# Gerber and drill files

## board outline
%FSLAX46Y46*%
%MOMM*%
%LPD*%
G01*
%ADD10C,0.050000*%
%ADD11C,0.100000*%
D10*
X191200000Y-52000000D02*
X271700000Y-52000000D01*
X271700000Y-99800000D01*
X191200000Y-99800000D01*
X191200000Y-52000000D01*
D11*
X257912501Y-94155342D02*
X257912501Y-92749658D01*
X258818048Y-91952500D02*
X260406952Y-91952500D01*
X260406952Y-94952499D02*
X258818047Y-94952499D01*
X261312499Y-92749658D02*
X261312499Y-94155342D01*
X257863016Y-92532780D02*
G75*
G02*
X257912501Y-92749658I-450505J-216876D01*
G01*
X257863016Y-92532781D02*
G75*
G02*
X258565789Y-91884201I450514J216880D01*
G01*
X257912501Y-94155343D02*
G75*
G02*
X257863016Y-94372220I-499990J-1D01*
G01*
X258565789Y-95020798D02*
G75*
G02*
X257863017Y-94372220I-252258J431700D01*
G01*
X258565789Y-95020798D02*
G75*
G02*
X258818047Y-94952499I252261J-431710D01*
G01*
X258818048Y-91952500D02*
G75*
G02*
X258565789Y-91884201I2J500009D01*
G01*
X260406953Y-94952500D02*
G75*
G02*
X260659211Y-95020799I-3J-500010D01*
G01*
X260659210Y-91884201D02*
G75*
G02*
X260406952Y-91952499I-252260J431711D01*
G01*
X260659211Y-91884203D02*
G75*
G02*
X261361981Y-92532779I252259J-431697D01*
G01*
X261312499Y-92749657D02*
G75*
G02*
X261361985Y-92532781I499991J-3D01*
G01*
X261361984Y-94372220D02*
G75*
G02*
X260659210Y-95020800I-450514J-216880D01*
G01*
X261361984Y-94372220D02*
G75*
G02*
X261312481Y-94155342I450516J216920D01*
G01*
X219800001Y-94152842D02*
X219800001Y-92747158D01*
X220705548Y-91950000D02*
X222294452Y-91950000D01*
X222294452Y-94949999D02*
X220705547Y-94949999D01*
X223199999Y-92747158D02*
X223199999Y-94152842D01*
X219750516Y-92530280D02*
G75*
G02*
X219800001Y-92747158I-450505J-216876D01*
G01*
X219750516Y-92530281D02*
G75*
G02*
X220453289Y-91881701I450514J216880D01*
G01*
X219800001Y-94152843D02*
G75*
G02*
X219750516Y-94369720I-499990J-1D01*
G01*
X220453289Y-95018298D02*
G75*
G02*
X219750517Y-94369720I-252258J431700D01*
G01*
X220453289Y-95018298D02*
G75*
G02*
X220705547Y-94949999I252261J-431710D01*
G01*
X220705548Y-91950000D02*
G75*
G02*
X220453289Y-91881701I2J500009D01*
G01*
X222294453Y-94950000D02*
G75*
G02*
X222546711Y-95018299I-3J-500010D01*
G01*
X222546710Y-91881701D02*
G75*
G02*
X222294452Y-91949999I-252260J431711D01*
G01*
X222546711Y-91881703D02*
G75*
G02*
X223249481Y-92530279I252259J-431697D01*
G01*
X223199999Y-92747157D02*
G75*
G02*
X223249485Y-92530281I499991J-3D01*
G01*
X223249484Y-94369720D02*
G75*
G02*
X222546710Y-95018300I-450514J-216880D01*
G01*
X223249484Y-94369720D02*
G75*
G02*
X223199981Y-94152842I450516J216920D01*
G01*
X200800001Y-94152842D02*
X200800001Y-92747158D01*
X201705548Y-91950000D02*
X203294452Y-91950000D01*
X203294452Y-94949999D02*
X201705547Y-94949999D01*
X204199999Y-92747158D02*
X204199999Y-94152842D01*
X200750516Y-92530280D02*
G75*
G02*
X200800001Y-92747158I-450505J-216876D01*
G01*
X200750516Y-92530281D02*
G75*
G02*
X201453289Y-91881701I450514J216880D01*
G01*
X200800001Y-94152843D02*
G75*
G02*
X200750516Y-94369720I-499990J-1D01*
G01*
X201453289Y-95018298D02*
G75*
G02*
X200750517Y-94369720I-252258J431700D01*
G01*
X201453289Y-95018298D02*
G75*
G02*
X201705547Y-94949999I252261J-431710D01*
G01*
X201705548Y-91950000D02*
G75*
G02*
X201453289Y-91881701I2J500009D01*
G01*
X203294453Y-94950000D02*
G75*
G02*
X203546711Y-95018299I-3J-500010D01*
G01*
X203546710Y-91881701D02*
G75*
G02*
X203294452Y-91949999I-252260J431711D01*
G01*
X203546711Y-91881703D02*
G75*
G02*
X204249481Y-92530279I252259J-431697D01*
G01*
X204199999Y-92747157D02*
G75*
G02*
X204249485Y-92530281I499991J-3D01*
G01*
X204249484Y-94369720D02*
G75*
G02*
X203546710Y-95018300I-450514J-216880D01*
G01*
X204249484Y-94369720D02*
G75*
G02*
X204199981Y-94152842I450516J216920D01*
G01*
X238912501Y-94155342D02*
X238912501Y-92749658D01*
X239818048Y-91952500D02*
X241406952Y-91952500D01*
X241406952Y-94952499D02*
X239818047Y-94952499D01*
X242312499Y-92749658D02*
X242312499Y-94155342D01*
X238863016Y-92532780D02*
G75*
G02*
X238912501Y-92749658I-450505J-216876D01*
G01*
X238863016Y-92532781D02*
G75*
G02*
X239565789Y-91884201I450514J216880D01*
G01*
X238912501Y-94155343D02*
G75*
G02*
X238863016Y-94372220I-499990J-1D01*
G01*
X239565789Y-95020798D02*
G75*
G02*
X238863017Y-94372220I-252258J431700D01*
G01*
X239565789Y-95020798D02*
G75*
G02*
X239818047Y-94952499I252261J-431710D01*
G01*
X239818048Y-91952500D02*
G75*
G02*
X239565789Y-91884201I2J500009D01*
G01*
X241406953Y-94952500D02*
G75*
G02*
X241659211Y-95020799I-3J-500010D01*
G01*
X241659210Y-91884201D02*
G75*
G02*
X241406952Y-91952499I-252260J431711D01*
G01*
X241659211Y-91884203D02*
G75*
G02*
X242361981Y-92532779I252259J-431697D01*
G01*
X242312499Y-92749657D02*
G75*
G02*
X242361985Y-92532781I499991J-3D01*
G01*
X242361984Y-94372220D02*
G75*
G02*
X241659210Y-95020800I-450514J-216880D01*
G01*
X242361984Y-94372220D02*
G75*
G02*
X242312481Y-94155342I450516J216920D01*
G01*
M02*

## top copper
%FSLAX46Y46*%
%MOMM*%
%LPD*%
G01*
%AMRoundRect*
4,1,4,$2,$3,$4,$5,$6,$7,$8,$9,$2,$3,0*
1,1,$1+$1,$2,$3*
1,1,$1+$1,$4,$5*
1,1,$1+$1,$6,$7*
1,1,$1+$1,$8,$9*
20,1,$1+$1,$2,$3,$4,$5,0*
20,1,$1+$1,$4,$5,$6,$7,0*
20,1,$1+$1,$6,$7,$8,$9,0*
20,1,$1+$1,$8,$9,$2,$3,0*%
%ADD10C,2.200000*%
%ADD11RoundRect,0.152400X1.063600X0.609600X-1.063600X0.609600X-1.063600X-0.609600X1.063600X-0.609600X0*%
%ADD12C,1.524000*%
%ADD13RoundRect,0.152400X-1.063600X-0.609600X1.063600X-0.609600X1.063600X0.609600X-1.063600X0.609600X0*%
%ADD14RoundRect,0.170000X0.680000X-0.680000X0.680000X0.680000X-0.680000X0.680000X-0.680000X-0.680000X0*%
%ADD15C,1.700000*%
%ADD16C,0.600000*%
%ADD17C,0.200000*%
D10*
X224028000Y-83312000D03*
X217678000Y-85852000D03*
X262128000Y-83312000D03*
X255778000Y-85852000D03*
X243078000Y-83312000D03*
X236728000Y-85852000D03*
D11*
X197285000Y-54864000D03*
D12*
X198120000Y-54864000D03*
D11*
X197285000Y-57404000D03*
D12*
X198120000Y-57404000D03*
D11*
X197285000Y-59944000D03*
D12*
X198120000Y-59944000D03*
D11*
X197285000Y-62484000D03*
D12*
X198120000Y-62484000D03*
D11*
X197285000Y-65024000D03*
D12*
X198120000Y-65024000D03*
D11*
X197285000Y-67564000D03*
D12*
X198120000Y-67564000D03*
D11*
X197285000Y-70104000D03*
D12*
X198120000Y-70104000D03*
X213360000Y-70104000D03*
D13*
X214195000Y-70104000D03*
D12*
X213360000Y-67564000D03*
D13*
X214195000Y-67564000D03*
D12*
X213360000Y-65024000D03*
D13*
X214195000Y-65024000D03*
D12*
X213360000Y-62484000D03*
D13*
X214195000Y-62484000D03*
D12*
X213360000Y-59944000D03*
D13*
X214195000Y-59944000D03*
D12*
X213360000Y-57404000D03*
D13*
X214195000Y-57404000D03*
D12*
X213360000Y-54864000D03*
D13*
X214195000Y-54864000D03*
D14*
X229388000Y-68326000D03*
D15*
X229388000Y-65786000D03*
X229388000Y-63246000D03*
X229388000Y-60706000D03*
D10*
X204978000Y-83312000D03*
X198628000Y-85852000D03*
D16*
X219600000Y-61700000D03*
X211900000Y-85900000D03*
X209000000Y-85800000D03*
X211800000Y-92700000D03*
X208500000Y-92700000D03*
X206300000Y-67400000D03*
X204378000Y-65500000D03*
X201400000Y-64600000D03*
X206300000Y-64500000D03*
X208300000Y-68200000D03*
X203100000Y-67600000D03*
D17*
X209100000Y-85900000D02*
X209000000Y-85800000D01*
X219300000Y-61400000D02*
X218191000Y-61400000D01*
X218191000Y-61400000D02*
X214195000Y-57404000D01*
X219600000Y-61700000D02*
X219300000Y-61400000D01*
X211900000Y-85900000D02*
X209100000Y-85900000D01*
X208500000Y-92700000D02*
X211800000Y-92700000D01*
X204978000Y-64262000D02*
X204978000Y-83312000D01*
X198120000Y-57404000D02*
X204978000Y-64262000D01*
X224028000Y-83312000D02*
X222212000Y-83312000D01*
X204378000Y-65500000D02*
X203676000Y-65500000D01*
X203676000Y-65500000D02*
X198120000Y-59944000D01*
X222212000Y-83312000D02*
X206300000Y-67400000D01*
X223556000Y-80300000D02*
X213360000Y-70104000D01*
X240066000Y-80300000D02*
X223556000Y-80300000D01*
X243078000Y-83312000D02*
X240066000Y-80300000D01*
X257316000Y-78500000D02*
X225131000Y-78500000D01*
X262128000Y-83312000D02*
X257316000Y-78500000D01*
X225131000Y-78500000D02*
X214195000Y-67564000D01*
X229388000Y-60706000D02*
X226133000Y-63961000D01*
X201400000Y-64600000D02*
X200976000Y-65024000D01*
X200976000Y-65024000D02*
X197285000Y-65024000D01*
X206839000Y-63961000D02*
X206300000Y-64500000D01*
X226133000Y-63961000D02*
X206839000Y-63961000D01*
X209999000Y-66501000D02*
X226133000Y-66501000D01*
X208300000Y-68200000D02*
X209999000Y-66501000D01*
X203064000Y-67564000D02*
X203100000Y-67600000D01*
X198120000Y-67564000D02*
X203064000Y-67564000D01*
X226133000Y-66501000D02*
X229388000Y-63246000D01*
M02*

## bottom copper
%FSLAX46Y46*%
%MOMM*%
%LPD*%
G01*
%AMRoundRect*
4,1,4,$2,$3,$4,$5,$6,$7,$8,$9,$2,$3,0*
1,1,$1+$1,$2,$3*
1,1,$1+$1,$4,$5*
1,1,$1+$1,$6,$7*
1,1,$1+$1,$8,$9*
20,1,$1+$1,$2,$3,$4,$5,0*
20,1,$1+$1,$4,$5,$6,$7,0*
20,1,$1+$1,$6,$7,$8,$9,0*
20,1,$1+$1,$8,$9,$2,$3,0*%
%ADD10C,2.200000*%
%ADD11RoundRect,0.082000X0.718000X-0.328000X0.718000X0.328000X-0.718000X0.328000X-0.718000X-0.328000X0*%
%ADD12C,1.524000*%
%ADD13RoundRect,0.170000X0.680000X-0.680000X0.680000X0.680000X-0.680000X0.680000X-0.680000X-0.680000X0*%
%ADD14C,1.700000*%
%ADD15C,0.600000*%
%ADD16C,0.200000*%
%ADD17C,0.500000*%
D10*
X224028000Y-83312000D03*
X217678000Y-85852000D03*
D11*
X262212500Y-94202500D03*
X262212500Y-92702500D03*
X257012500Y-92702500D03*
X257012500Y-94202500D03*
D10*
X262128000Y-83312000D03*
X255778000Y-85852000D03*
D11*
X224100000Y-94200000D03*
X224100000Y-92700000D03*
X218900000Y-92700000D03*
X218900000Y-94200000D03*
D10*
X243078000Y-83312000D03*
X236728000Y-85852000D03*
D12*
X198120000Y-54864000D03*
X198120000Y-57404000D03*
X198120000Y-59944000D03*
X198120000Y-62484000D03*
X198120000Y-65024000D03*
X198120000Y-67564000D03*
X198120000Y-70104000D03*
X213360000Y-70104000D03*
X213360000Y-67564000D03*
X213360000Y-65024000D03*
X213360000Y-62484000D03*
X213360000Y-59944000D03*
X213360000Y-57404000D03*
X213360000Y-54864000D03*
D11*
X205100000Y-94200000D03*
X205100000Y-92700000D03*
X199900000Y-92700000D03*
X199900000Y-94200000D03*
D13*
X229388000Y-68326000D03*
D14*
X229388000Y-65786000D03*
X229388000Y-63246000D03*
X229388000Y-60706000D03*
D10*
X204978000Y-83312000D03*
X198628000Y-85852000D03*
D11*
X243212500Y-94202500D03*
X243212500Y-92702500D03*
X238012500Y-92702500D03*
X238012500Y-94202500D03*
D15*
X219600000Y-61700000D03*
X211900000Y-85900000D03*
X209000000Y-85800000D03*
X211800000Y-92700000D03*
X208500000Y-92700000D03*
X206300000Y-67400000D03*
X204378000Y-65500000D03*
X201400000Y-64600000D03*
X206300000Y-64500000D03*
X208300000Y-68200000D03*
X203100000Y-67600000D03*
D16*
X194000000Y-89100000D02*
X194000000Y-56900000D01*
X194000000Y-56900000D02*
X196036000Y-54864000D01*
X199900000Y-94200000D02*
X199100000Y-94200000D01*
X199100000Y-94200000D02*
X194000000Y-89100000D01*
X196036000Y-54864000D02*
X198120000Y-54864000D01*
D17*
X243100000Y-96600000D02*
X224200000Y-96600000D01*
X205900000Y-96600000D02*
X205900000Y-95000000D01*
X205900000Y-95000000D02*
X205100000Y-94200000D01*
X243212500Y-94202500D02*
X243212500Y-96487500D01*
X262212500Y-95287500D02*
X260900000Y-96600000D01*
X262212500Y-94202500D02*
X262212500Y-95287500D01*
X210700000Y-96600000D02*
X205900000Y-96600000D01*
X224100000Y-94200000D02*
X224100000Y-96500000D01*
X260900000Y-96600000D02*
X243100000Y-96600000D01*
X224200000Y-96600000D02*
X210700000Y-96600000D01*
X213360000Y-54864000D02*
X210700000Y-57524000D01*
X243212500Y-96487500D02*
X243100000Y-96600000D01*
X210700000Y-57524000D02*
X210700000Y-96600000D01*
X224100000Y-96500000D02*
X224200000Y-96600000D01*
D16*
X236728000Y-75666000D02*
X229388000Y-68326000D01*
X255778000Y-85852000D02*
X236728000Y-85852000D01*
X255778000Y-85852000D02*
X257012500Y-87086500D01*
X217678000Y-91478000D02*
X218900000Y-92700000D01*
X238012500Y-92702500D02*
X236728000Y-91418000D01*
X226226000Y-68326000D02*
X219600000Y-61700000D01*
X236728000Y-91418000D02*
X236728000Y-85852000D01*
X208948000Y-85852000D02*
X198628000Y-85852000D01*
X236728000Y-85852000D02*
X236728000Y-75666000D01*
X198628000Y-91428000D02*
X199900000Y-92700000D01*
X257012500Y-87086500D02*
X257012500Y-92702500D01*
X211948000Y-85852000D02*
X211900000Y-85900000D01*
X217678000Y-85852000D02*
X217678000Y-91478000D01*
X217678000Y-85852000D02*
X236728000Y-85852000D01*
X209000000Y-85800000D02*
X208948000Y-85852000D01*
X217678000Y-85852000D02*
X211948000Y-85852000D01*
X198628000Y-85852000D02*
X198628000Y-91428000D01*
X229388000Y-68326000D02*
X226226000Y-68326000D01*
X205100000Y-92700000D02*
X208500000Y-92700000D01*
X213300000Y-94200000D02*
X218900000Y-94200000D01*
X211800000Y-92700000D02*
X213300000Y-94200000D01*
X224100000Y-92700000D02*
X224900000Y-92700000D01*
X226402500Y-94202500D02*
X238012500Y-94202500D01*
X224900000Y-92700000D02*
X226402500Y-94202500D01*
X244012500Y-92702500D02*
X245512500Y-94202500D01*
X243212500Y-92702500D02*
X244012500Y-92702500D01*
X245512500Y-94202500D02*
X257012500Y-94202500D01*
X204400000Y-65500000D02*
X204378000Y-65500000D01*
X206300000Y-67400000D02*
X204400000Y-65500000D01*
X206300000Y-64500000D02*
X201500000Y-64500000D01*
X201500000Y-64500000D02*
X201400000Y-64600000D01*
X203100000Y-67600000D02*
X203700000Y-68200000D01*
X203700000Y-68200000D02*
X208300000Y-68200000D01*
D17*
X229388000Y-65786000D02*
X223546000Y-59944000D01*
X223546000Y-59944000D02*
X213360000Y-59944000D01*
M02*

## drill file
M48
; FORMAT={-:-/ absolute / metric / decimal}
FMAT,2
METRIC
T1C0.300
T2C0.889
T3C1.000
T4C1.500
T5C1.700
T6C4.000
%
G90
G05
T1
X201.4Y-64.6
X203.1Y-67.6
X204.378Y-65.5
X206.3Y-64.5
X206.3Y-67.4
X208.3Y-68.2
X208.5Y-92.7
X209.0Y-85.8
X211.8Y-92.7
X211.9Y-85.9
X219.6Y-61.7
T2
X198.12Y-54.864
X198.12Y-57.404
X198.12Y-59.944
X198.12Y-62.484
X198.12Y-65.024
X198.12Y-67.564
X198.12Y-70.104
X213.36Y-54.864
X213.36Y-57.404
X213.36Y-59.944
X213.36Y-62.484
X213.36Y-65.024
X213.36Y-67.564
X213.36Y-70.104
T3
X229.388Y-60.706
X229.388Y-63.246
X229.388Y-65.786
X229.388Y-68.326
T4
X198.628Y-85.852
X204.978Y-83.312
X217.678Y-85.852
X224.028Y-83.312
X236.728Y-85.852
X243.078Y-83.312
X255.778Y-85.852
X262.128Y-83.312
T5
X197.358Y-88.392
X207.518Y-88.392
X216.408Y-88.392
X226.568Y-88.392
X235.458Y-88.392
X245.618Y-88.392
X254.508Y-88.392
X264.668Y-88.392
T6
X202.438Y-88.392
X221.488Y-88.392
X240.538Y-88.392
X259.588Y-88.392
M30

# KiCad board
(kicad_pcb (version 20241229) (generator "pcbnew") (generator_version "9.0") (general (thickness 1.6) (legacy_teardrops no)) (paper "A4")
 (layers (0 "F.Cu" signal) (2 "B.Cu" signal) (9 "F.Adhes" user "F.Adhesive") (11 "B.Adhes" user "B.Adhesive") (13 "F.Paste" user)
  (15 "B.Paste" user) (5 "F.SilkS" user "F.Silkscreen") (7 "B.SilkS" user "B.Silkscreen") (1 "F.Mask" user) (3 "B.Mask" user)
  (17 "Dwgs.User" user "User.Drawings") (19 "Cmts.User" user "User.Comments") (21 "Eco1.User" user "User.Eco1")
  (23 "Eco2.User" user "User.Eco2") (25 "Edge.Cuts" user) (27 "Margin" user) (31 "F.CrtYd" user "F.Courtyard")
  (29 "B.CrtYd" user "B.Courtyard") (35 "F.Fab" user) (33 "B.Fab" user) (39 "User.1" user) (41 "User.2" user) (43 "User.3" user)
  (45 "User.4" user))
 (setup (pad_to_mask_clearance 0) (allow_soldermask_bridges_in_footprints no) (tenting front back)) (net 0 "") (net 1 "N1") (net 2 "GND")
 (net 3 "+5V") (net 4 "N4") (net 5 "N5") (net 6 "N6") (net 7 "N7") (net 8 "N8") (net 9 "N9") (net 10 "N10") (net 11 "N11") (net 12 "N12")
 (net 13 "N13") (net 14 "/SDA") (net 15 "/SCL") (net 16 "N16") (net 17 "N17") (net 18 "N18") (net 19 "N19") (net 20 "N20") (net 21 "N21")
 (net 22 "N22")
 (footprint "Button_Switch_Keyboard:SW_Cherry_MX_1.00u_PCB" (layer "F.Cu") (at 224.028 83.312)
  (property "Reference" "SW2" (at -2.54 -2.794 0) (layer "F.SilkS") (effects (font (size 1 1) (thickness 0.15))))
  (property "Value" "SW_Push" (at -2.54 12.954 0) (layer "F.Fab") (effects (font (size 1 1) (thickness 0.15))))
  (pad "" np_thru_hole circle (at -7.62 5.08) (size 1.7 1.7) (drill 1.7) (layers "*.Cu" "*.Mask"))
  (pad "" np_thru_hole circle (at -2.54 5.08) (size 4 4) (drill 4) (layers "*.Cu" "*.Mask"))
  (pad "" np_thru_hole circle (at 2.54 5.08) (size 1.7 1.7) (drill 1.7) (layers "*.Cu" "*.Mask"))
  (pad "1" thru_hole circle (at 0 0) (size 2.2 2.2) (drill 1.5) (layers "*.Cu" "*.Mask") (remove_unused_layers no) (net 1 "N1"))
  (pad "2" thru_hole circle (at -6.35 2.54) (size 2.2 2.2) (drill 1.5) (layers "*.Cu" "*.Mask") (remove_unused_layers no) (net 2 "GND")))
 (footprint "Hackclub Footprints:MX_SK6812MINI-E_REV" (layer "F.Cu") (at 259.6125 88.3725)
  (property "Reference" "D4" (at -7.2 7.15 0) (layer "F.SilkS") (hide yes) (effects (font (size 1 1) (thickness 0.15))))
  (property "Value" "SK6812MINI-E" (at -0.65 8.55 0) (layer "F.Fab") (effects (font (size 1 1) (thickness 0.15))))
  (fp_line (start -1.699999 5.782842) (end -1.699999 4.377158) (stroke (width 0.1) (type solid)) (layer "Edge.Cuts"))
  (fp_line (start -0.794452 3.58) (end 0.794452 3.58) (stroke (width 0.1) (type solid)) (layer "Edge.Cuts"))
  (fp_line (start 0.794452 6.579999) (end -0.794453 6.579999) (stroke (width 0.1) (type solid)) (layer "Edge.Cuts"))
  (fp_line (start 1.699999 4.377158) (end 1.699999 5.782842) (stroke (width 0.1) (type solid)) (layer "Edge.Cuts"))
  (fp_arc (start -1.749484 4.16028) (mid -1.712527 4.265932) (end -1.699999 4.377158) (stroke (width 0.1) (type solid)) (layer "Edge.Cuts"))
  (fp_arc (start -1.749484 4.160281) (mid -1.638072 3.575965) (end -1.046711 3.511701) (stroke (width 0.1) (type solid)) (layer "Edge.Cuts"))
  (fp_arc (start -1.699999 5.782843) (mid -1.712527 5.894068) (end -1.749484 5.99972) (stroke (width 0.1) (type solid)) (layer "Edge.Cuts"))
  (fp_arc (start -1.046711 6.648298) (mid -1.638071 6.584034) (end -1.749484 5.99972) (stroke (width 0.1) (type solid)) (layer "Edge.Cuts"))
  (fp_arc (start -1.046711 6.648298) (mid -0.925123 6.597376) (end -0.794453 6.579999) (stroke (width 0.1) (type solid)) (layer "Edge.Cuts"))
  (fp_arc (start -0.794452 3.58) (mid -0.925123 3.562623) (end -1.046711 3.511701) (stroke (width 0.1) (type solid)) (layer "Edge.Cuts"))
  (fp_arc (start 0.794453 6.58) (mid 0.925123 6.597377) (end 1.046711 6.648299) (stroke (width 0.1) (type solid)) (layer "Edge.Cuts"))
  (fp_arc (start 1.04671 3.511701) (mid 0.925122 3.562623) (end 0.794452 3.58) (stroke (width 0.1) (type solid)) (layer "Edge.Cuts"))
  (fp_arc (start 1.046711 3.511703) (mid 1.63807 3.575966) (end 1.749484 4.16028) (stroke (width 0.1) (type solid)) (layer "Edge.Cuts"))
  (fp_arc (start 1.699999 4.377157) (mid 1.712527 4.265932) (end 1.749484 4.16028) (stroke (width 0.1) (type solid)) (layer "Edge.Cuts"))
  (fp_arc (start 1.749484 5.99972) (mid 1.638071 6.584035) (end 1.046711 6.648299) (stroke (width 0.1) (type solid)) (layer "Edge.Cuts"))
  (fp_arc (start 1.749484 5.99972) (mid 1.712527 5.894068) (end 1.699999 5.782842) (stroke (width 0.1) (type solid)) (layer "Edge.Cuts"))
  (pad "1" smd roundrect (at 2.6 5.83 90) (size 0.82 1.6) (layers "B.Cu" "B.Mask" "B.Paste") (roundrect_rratio 0.1) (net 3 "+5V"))
  (pad "2" smd roundrect (at 2.6 4.33 90) (size 0.82 1.6) (layers "B.Cu" "B.Mask" "B.Paste") (roundrect_rratio 0.1) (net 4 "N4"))
  (pad "3" smd roundrect (at -2.6 4.33 90) (size 0.82 1.6) (layers "B.Cu" "B.Mask" "B.Paste") (roundrect_rratio 0.1) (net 2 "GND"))
  (pad "4" smd roundrect (at -2.6 5.83 90) (size 0.82 1.6) (layers "B.Cu" "B.Mask" "B.Paste") (roundrect_rratio 0.1) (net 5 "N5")))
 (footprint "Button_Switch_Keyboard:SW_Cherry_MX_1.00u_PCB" (layer "F.Cu") (at 262.128 83.312)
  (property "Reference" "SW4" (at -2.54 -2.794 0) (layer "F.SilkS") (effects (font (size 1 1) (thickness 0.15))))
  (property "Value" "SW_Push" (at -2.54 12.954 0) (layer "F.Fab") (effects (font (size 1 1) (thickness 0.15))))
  (pad "" np_thru_hole circle (at -7.62 5.08) (size 1.7 1.7) (drill 1.7) (layers "*.Cu" "*.Mask"))
  (pad "" np_thru_hole circle (at -2.54 5.08) (size 4 4) (drill 4) (layers "*.Cu" "*.Mask"))
  (pad "" np_thru_hole circle (at 2.54 5.08) (size 1.7 1.7) (drill 1.7) (layers "*.Cu" "*.Mask"))
  (pad "1" thru_hole circle (at 0 0) (size 2.2 2.2) (drill 1.5) (layers "*.Cu" "*.Mask") (remove_unused_layers no) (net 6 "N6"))
  (pad "2" thru_hole circle (at -6.35 2.54) (size 2.2 2.2) (drill 1.5) (layers "*.Cu" "*.Mask") (remove_unused_layers no) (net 2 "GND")))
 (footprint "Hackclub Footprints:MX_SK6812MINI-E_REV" (layer "F.Cu") (at 221.5 88.37)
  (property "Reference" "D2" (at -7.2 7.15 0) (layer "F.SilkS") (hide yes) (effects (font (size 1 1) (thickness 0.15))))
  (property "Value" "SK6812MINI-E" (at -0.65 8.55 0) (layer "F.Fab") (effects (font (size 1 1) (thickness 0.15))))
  (fp_line (start -1.699999 5.782842) (end -1.699999 4.377158) (stroke (width 0.1) (type solid)) (layer "Edge.Cuts"))
  (fp_line (start -0.794452 3.58) (end 0.794452 3.58) (stroke (width 0.1) (type solid)) (layer "Edge.Cuts"))
  (fp_line (start 0.794452 6.579999) (end -0.794453 6.579999) (stroke (width 0.1) (type solid)) (layer "Edge.Cuts"))
  (fp_line (start 1.699999 4.377158) (end 1.699999 5.782842) (stroke (width 0.1) (type solid)) (layer "Edge.Cuts"))
  (fp_arc (start -1.749484 4.16028) (mid -1.712527 4.265932) (end -1.699999 4.377158) (stroke (width 0.1) (type solid)) (layer "Edge.Cuts"))
  (fp_arc (start -1.749484 4.160281) (mid -1.638072 3.575965) (end -1.046711 3.511701) (stroke (width 0.1) (type solid)) (layer "Edge.Cuts"))
  (fp_arc (start -1.699999 5.782843) (mid -1.712527 5.894068) (end -1.749484 5.99972) (stroke (width 0.1) (type solid)) (layer "Edge.Cuts"))
  (fp_arc (start -1.046711 6.648298) (mid -1.638071 6.584034) (end -1.749484 5.99972) (stroke (width 0.1) (type solid)) (layer "Edge.Cuts"))
  (fp_arc (start -1.046711 6.648298) (mid -0.925123 6.597376) (end -0.794453 6.579999) (stroke (width 0.1) (type solid)) (layer "Edge.Cuts"))
  (fp_arc (start -0.794452 3.58) (mid -0.925123 3.562623) (end -1.046711 3.511701) (stroke (width 0.1) (type solid)) (layer "Edge.Cuts"))
  (fp_arc (start 0.794453 6.58) (mid 0.925123 6.597377) (end 1.046711 6.648299) (stroke (width 0.1) (type solid)) (layer "Edge.Cuts"))
  (fp_arc (start 1.04671 3.511701) (mid 0.925122 3.562623) (end 0.794452 3.58) (stroke (width 0.1) (type solid)) (layer "Edge.Cuts"))
  (fp_arc (start 1.046711 3.511703) (mid 1.63807 3.575966) (end 1.749484 4.16028) (stroke (width 0.1) (type solid)) (layer "Edge.Cuts"))
  (fp_arc (start 1.699999 4.377157) (mid 1.712527 4.265932) (end 1.749484 4.16028) (stroke (width 0.1) (type solid)) (layer "Edge.Cuts"))
  (fp_arc (start 1.749484 5.99972) (mid 1.638071 6.584035) (end 1.046711 6.648299) (stroke (width 0.1) (type solid)) (layer "Edge.Cuts"))
  (fp_arc (start 1.749484 5.99972) (mid 1.712527 5.894068) (end 1.699999 5.782842) (stroke (width 0.1) (type solid)) (layer "Edge.Cuts"))
  (pad "1" smd roundrect (at 2.6 5.83 90) (size 0.82 1.6) (layers "B.Cu" "B.Mask" "B.Paste") (roundrect_rratio 0.1) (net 3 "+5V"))
  (pad "2" smd roundrect (at 2.6 4.33 90) (size 0.82 1.6) (layers "B.Cu" "B.Mask" "B.Paste") (roundrect_rratio 0.1) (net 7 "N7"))
  (pad "3" smd roundrect (at -2.6 4.33 90) (size 0.82 1.6) (layers "B.Cu" "B.Mask" "B.Paste") (roundrect_rratio 0.1) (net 2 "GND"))
  (pad "4" smd roundrect (at -2.6 5.83 90) (size 0.82 1.6) (layers "B.Cu" "B.Mask" "B.Paste") (roundrect_rratio 0.1) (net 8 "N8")))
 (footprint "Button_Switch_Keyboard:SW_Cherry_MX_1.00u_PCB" (layer "F.Cu") (at 243.078 83.312)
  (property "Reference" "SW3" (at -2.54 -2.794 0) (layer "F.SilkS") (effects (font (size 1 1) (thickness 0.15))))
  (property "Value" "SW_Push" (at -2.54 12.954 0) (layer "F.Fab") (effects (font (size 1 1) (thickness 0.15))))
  (pad "" np_thru_hole circle (at -7.62 5.08) (size 1.7 1.7) (drill 1.7) (layers "*.Cu" "*.Mask"))
  (pad "" np_thru_hole circle (at -2.54 5.08) (size 4 4) (drill 4) (layers "*.Cu" "*.Mask"))
  (pad "" np_thru_hole circle (at 2.54 5.08) (size 1.7 1.7) (drill 1.7) (layers "*.Cu" "*.Mask"))
  (pad "1" thru_hole circle (at 0 0) (size 2.2 2.2) (drill 1.5) (layers "*.Cu" "*.Mask") (remove_unused_layers no) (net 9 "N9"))
  (pad "2" thru_hole circle (at -6.35 2.54) (size 2.2 2.2) (drill 1.5) (layers "*.Cu" "*.Mask") (remove_unused_layers no) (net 2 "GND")))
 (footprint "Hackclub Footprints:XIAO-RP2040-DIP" (layer "F.Cu") (at 205.74 62.484)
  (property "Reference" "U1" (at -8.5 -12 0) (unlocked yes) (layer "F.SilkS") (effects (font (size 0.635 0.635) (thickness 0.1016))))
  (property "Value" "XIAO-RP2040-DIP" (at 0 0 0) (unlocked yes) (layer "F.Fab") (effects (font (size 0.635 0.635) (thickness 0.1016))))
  (pad "1" smd roundrect (at -8.455 -7.62 180) (size 2.432 1.524) (layers "F.Cu" "F.Mask") (roundrect_rratio 0.1) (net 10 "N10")
   (thermal_bridge_angle 45))
  (pad "1" thru_hole circle (at -7.62 -7.62 180) (size 1.524 1.524) (drill 0.889) (layers "*.Cu" "*.Mask") (remove_unused_layers no)
   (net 10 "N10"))
  (pad "2" smd roundrect (at -8.455 -5.08 180) (size 2.432 1.524) (layers "F.Cu" "F.Mask") (roundrect_rratio 0.1) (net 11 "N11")
   (thermal_bridge_angle 45))
  (pad "2" thru_hole circle (at -7.62 -5.08 180) (size 1.524 1.524) (drill 0.889) (layers "*.Cu" "*.Mask") (remove_unused_layers no)
   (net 11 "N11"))
  (pad "3" smd roundrect (at -8.455 -2.54 180) (size 2.432 1.524) (layers "F.Cu" "F.Mask") (roundrect_rratio 0.1) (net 1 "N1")
   (thermal_bridge_angle 45))
  (pad "3" thru_hole circle (at -7.62 -2.54 180) (size 1.524 1.524) (drill 0.889) (layers "*.Cu" "*.Mask") (remove_unused_layers no)
   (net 1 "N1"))
  (pad "4" smd roundrect (at -8.455 0 180) (size 2.432 1.524) (layers "F.Cu" "F.Mask") (roundrect_rratio 0.1) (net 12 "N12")
   (thermal_bridge_angle 45))
  (pad "4" thru_hole circle (at -7.62 0 180) (size 1.524 1.524) (drill 0.889) (layers "*.Cu" "*.Mask") (remove_unused_layers no)
   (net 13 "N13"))
  (pad "5" smd roundrect (at -8.455 2.54 180) (size 2.432 1.524) (layers "F.Cu" "F.Mask") (roundrect_rratio 0.1) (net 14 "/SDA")
   (thermal_bridge_angle 45))
  (pad "5" thru_hole circle (at -7.62 2.54 180) (size 1.524 1.524) (drill 0.889) (layers "*.Cu" "*.Mask") (remove_unused_layers no)
   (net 14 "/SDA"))
  (pad "6" smd roundrect (at -8.455 5.08 180) (size 2.432 1.524) (layers "F.Cu" "F.Mask") (roundrect_rratio 0.1) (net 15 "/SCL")
   (thermal_bridge_angle 45))
  (pad "6" thru_hole circle (at -7.62 5.08 180) (size 1.524 1.524) (drill 0.889) (layers "*.Cu" "*.Mask") (remove_unused_layers no)
   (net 15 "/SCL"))
  (pad "7" smd roundrect (at -8.455 7.62 180) (size 2.432 1.524) (layers "F.Cu" "F.Mask") (roundrect_rratio 0.1) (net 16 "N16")
   (thermal_bridge_angle 45))
  (pad "7" thru_hole circle (at -7.62 7.62 180) (size 1.524 1.524) (drill 0.889) (layers "*.Cu" "*.Mask") (remove_unused_layers no)
   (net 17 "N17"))
  (pad "8" thru_hole circle (at 7.62 7.62) (size 1.524 1.524) (drill 0.889) (layers "*.Cu" "*.Mask") (remove_unused_layers no) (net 9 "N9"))
  (pad "8" smd roundrect (at 8.455 7.62) (size 2.432 1.524) (layers "F.Cu" "F.Mask") (roundrect_rratio 0.1) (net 9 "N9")
   (thermal_bridge_angle 45))
  (pad "9" thru_hole circle (at 7.62 5.08) (size 1.524 1.524) (drill 0.889) (layers "*.Cu" "*.Mask") (remove_unused_layers no) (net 6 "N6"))
  (pad "9" smd roundrect (at 8.455 5.08) (size 2.432 1.524) (layers "F.Cu" "F.Mask") (roundrect_rratio 0.1) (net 6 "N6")
   (thermal_bridge_angle 45))
  (pad "10" thru_hole circle (at 7.62 2.54) (size 1.524 1.524) (drill 0.889) (layers "*.Cu" "*.Mask") (remove_unused_layers no)
   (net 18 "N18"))
  (pad "10" smd roundrect (at 8.455 2.54) (size 2.432 1.524) (layers "F.Cu" "F.Mask") (roundrect_rratio 0.1) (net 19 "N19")
   (thermal_bridge_angle 45))
  (pad "11" thru_hole circle (at 7.62 0) (size 1.524 1.524) (drill 0.889) (layers "*.Cu" "*.Mask") (remove_unused_layers no) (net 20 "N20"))
  (pad "11" smd roundrect (at 8.455 0) (size 2.432 1.524) (layers "F.Cu" "F.Mask") (roundrect_rratio 0.1) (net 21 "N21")
   (thermal_bridge_angle 45))
  (pad "12" thru_hole circle (at 7.62 -2.54) (size 1.524 1.524) (drill 0.889) (layers "*.Cu" "*.Mask") (remove_unused_layers no)
   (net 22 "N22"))
  (pad "12" smd roundrect (at 8.455 -2.54) (size 2.432 1.524) (layers "F.Cu" "F.Mask") (roundrect_rratio 0.1) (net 22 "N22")
   (thermal_bridge_angle 45))
  (pad "13" thru_hole circle (at 7.62 -5.08) (size 1.524 1.524) (drill 0.889) (layers "*.Cu" "*.Mask") (remove_unused_layers no)
   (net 2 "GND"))
  (pad "13" smd roundrect (at 8.455 -5.08) (size 2.432 1.524) (layers "F.Cu" "F.Mask") (roundrect_rratio 0.1) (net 2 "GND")
   (thermal_bridge_angle 45))
  (pad "14" thru_hole circle (at 7.62 -7.62) (size 1.524 1.524) (drill 0.889) (layers "*.Cu" "*.Mask") (remove_unused_layers no)
   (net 3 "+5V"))
  (pad "14" smd roundrect (at 8.455 -7.62) (size 2.432 1.524) (layers "F.Cu" "F.Mask") (roundrect_rratio 0.1) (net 3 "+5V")
   (thermal_bridge_angle 45)))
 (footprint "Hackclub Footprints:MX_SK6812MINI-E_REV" (layer "F.Cu") (at 202.5 88.37)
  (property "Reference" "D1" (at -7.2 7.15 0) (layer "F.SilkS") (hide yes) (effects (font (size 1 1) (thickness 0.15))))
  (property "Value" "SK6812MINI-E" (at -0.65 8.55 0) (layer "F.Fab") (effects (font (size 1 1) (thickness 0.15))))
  (fp_line (start -1.699999 5.782842) (end -1.699999 4.377158) (stroke (width 0.1) (type solid)) (layer "Edge.Cuts"))
  (fp_line (start -0.794452 3.58) (end 0.794452 3.58) (stroke (width 0.1) (type solid)) (layer "Edge.Cuts"))
  (fp_line (start 0.794452 6.579999) (end -0.794453 6.579999) (stroke (width 0.1) (type solid)) (layer "Edge.Cuts"))
  (fp_line (start 1.699999 4.377158) (end 1.699999 5.782842) (stroke (width 0.1) (type solid)) (layer "Edge.Cuts"))
  (fp_arc (start -1.749484 4.16028) (mid -1.712527 4.265932) (end -1.699999 4.377158) (stroke (width 0.1) (type solid)) (layer "Edge.Cuts"))
  (fp_arc (start -1.749484 4.160281) (mid -1.638072 3.575965) (end -1.046711 3.511701) (stroke (width 0.1) (type solid)) (layer "Edge.Cuts"))
  (fp_arc (start -1.699999 5.782843) (mid -1.712527 5.894068) (end -1.749484 5.99972) (stroke (width 0.1) (type solid)) (layer "Edge.Cuts"))
  (fp_arc (start -1.046711 6.648298) (mid -1.638071 6.584034) (end -1.749484 5.99972) (stroke (width 0.1) (type solid)) (layer "Edge.Cuts"))
  (fp_arc (start -1.046711 6.648298) (mid -0.925123 6.597376) (end -0.794453 6.579999) (stroke (width 0.1) (type solid)) (layer "Edge.Cuts"))
  (fp_arc (start -0.794452 3.58) (mid -0.925123 3.562623) (end -1.046711 3.511701) (stroke (width 0.1) (type solid)) (layer "Edge.Cuts"))
  (fp_arc (start 0.794453 6.58) (mid 0.925123 6.597377) (end 1.046711 6.648299) (stroke (width 0.1) (type solid)) (layer "Edge.Cuts"))
  (fp_arc (start 1.04671 3.511701) (mid 0.925122 3.562623) (end 0.794452 3.58) (stroke (width 0.1) (type solid)) (layer "Edge.Cuts"))
  (fp_arc (start 1.046711 3.511703) (mid 1.63807 3.575966) (end 1.749484 4.16028) (stroke (width 0.1) (type solid)) (layer "Edge.Cuts"))
  (fp_arc (start 1.699999 4.377157) (mid 1.712527 4.265932) (end 1.749484 4.16028) (stroke (width 0.1) (type solid)) (layer "Edge.Cuts"))
  (fp_arc (start 1.749484 5.99972) (mid 1.638071 6.584035) (end 1.046711 6.648299) (stroke (width 0.1) (type solid)) (layer "Edge.Cuts"))
  (fp_arc (start 1.749484 5.99972) (mid 1.712527 5.894068) (end 1.699999 5.782842) (stroke (width 0.1) (type solid)) (layer "Edge.Cuts"))
  (pad "1" smd roundrect (at 2.6 5.83 90) (size 0.82 1.6) (layers "B.Cu" "B.Mask" "B.Paste") (roundrect_rratio 0.1) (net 3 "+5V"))
  (pad "2" smd roundrect (at 2.6 4.33 90) (size 0.82 1.6) (layers "B.Cu" "B.Mask" "B.Paste") (roundrect_rratio 0.1) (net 8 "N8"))
  (pad "3" smd roundrect (at -2.6 4.33 90) (size 0.82 1.6) (layers "B.Cu" "B.Mask" "B.Paste") (roundrect_rratio 0.1) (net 2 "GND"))
  (pad "4" smd roundrect (at -2.6 5.83 90) (size 0.82 1.6) (layers "B.Cu" "B.Mask" "B.Paste") (roundrect_rratio 0.1) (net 10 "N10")))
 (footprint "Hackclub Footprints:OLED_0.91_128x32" (layer "F.Cu") (at 229.388 68.326 90)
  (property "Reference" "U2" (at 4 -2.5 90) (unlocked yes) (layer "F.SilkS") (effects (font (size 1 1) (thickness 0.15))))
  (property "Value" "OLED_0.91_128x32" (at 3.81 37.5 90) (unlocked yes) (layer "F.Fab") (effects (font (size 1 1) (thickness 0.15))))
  (pad "1" thru_hole roundrect (at 0 0 90) (size 1.7 1.7) (drill 1) (layers "*.Cu" "*.Mask") (remove_unused_layers no)
   (roundrect_rratio 0.1) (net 2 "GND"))
  (pad "2" thru_hole circle (at 2.54 0 90) (size 1.7 1.7) (drill 1) (layers "*.Cu" "*.Mask") (remove_unused_layers no) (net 22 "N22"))
  (pad "3" thru_hole circle (at 5.08 0 90) (size 1.7 1.7) (drill 1) (layers "*.Cu" "*.Mask") (remove_unused_layers no) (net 15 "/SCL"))
  (pad "4" thru_hole circle (at 7.62 0 90) (size 1.7 1.7) (drill 1) (layers "*.Cu" "*.Mask") (remove_unused_layers no) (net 14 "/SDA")))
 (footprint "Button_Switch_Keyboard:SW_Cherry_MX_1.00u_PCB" (layer "F.Cu") (at 204.978 83.312)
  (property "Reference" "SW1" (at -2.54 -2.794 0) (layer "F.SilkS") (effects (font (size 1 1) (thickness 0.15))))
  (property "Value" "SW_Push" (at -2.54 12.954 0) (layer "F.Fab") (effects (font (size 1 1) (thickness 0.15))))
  (pad "" np_thru_hole circle (at -7.62 5.08) (size 1.7 1.7) (drill 1.7) (layers "*.Cu" "*.Mask"))
  (pad "" np_thru_hole circle (at -2.54 5.08) (size 4 4) (drill 4) (layers "*.Cu" "*.Mask"))
  (pad "" np_thru_hole circle (at 2.54 5.08) (size 1.7 1.7) (drill 1.7) (layers "*.Cu" "*.Mask"))
  (pad "1" thru_hole circle (at 0 0) (size 2.2 2.2) (drill 1.5) (layers "*.Cu" "*.Mask") (remove_unused_layers no) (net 11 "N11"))
  (pad "2" thru_hole circle (at -6.35 2.54) (size 2.2 2.2) (drill 1.5) (layers "*.Cu" "*.Mask") (remove_unused_layers no) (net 2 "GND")))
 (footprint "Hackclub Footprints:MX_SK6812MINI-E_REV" (layer "F.Cu") (at 240.6125 88.3725)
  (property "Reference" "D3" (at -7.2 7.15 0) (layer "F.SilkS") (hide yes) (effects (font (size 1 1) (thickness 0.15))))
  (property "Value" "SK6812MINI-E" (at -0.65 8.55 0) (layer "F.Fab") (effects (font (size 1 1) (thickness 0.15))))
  (fp_line (start -1.699999 5.782842) (end -1.699999 4.377158) (stroke (width 0.1) (type solid)) (layer "Edge.Cuts"))
  (fp_line (start -0.794452 3.58) (end 0.794452 3.58) (stroke (width 0.1) (type solid)) (layer "Edge.Cuts"))
  (fp_line (start 0.794452 6.579999) (end -0.794453 6.579999) (stroke (width 0.1) (type solid)) (layer "Edge.Cuts"))
  (fp_line (start 1.699999 4.377158) (end 1.699999 5.782842) (stroke (width 0.1) (type solid)) (layer "Edge.Cuts"))
  (fp_arc (start -1.749484 4.16028) (mid -1.712527 4.265932) (end -1.699999 4.377158) (stroke (width 0.1) (type solid)) (layer "Edge.Cuts"))
  (fp_arc (start -1.749484 4.160281) (mid -1.638072 3.575965) (end -1.046711 3.511701) (stroke (width 0.1) (type solid)) (layer "Edge.Cuts"))
  (fp_arc (start -1.699999 5.782843) (mid -1.712527 5.894068) (end -1.749484 5.99972) (stroke (width 0.1) (type solid)) (layer "Edge.Cuts"))
  (fp_arc (start -1.046711 6.648298) (mid -1.638071 6.584034) (end -1.749484 5.99972) (stroke (width 0.1) (type solid)) (layer "Edge.Cuts"))
  (fp_arc (start -1.046711 6.648298) (mid -0.925123 6.597376) (end -0.794453 6.579999) (stroke (width 0.1) (type solid)) (layer "Edge.Cuts"))
  (fp_arc (start -0.794452 3.58) (mid -0.925123 3.562623) (end -1.046711 3.511701) (stroke (width 0.1) (type solid)) (layer "Edge.Cuts"))
  (fp_arc (start 0.794453 6.58) (mid 0.925123 6.597377) (end 1.046711 6.648299) (stroke (width 0.1) (type solid)) (layer "Edge.Cuts"))
  (fp_arc (start 1.04671 3.511701) (mid 0.925122 3.562623) (end 0.794452 3.58) (stroke (width 0.1) (type solid)) (layer "Edge.Cuts"))
  (fp_arc (start 1.046711 3.511703) (mid 1.63807 3.575966) (end 1.749484 4.16028) (stroke (width 0.1) (type solid)) (layer "Edge.Cuts"))
  (fp_arc (start 1.699999 4.377157) (mid 1.712527 4.265932) (end 1.749484 4.16028) (stroke (width 0.1) (type solid)) (layer "Edge.Cuts"))
  (fp_arc (start 1.749484 5.99972) (mid 1.638071 6.584035) (end 1.046711 6.648299) (stroke (width 0.1) (type solid)) (layer "Edge.Cuts"))
  (fp_arc (start 1.749484 5.99972) (mid 1.712527 5.894068) (end 1.699999 5.782842) (stroke (width 0.1) (type solid)) (layer "Edge.Cuts"))
  (pad "1" smd roundrect (at 2.6 5.83 90) (size 0.82 1.6) (layers "B.Cu" "B.Mask" "B.Paste") (roundrect_rratio 0.1) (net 3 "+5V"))
  (pad "2" smd roundrect (at 2.6 4.33 90) (size 0.82 1.6) (layers "B.Cu" "B.Mask" "B.Paste") (roundrect_rratio 0.1) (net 5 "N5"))
  (pad "3" smd roundrect (at -2.6 4.33 90) (size 0.82 1.6) (layers "B.Cu" "B.Mask" "B.Paste") (roundrect_rratio 0.1) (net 2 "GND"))
  (pad "4" smd roundrect (at -2.6 5.83 90) (size 0.82 1.6) (layers "B.Cu" "B.Mask" "B.Paste") (roundrect_rratio 0.1) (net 7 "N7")))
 (gr_rect (start 191.2 52) (end 271.7 99.8) (stroke (width 0.05) (type default)) (fill no) (layer "Edge.Cuts"))
 (segment (start 194 89.1) (end 194 56.9) (width 0.2) (layer "B.Cu") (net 10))
 (segment (start 194 56.9) (end 196.036 54.864) (width 0.2) (layer "B.Cu") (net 10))
 (segment (start 199.9 94.2) (end 199.1 94.2) (width 0.2) (layer "B.Cu") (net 10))
 (segment (start 199.1 94.2) (end 194 89.1) (width 0.2) (layer "B.Cu") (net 10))
 (segment (start 196.036 54.864) (end 198.12 54.864) (width 0.2) (layer "B.Cu") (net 10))
 (segment (start 243.1 96.6) (end 224.2 96.6) (width 0.5) (layer "B.Cu") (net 3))
 (segment (start 205.9 96.6) (end 205.9 95) (width 0.5) (layer "B.Cu") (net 3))
 (segment (start 205.9 95) (end 205.1 94.2) (width 0.5) (layer "B.Cu") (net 3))
 (segment (start 243.2125 94.2025) (end 243.2125 96.4875) (width 0.5) (layer "B.Cu") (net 3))
 (segment (start 262.2125 95.2875) (end 260.9 96.6) (width 0.5) (layer "B.Cu") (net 3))
 (segment (start 262.2125 94.2025) (end 262.2125 95.2875) (width 0.5) (layer "B.Cu") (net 3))
 (segment (start 210.7 96.6) (end 205.9 96.6) (width 0.5) (layer "B.Cu") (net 3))
 (segment (start 224.1 94.2) (end 224.1 96.5) (width 0.5) (layer "B.Cu") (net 3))
 (segment (start 260.9 96.6) (end 243.1 96.6) (width 0.5) (layer "B.Cu") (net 3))
 (segment (start 224.2 96.6) (end 210.7 96.6) (width 0.5) (layer "B.Cu") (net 3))
 (segment (start 213.36 54.864) (end 210.7 57.524) (width 0.5) (layer "B.Cu") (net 3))
 (segment (start 243.2125 96.4875) (end 243.1 96.6) (width 0.5) (layer "B.Cu") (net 3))
 (segment (start 210.7 57.524) (end 210.7 96.6) (width 0.5) (layer "B.Cu") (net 3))
 (segment (start 224.1 96.5) (end 224.2 96.6) (width 0.5) (layer "B.Cu") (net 3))
 (segment (start 209.1 85.9) (end 209 85.8) (width 0.2) (layer "F.Cu") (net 2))
 (segment (start 219.3 61.4) (end 218.191 61.4) (width 0.2) (layer "F.Cu") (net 2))
 (segment (start 218.191 61.4) (end 214.195 57.404) (width 0.2) (layer "F.Cu") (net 2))
 (segment (start 219.6 61.7) (end 219.3 61.4) (width 0.2) (layer "F.Cu") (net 2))
 (segment (start 211.9 85.9) (end 209.1 85.9) (width 0.2) (layer "F.Cu") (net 2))
 (via (at 219.6 61.7) (size 0.6) (drill 0.3) (layers "F.Cu" "B.Cu") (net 2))
 (via (at 211.9 85.9) (size 0.6) (drill 0.3) (layers "F.Cu" "B.Cu") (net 2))
 (via (at 209 85.8) (size 0.6) (drill 0.3) (layers "F.Cu" "B.Cu") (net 2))
 (segment (start 236.728 75.666) (end 229.388 68.326) (width 0.2) (layer "B.Cu") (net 2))
 (segment (start 255.778 85.852) (end 236.728 85.852) (width 0.2) (layer "B.Cu") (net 2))
 (segment (start 255.778 85.852) (end 257.0125 87.0865) (width 0.2) (layer "B.Cu") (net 2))
 (segment (start 217.678 91.478) (end 218.9 92.7) (width 0.2) (layer "B.Cu") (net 2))
 (segment (start 238.0125 92.7025) (end 236.728 91.418) (width 0.2) (layer "B.Cu") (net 2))
 (segment (start 226.226 68.326) (end 219.6 61.7) (width 0.2) (layer "B.Cu") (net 2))
 (segment (start 236.728 91.418) (end 236.728 85.852) (width 0.2) (layer "B.Cu") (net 2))
 (segment (start 208.948 85.852) (end 198.628 85.852) (width 0.2) (layer "B.Cu") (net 2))
 (segment (start 236.728 85.852) (end 236.728 75.666) (width 0.2) (layer "B.Cu") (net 2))
 (segment (start 198.628 91.428) (end 199.9 92.7) (width 0.2) (layer "B.Cu") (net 2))
 (segment (start 257.0125 87.0865) (end 257.0125 92.7025) (width 0.2) (layer "B.Cu") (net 2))
 (segment (start 211.948 85.852) (end 211.9 85.9) (width 0.2) (layer "B.Cu") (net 2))
 (segment (start 217.678 85.852) (end 217.678 91.478) (width 0.2) (layer "B.Cu") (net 2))
 (segment (start 217.678 85.852) (end 236.728 85.852) (width 0.2) (layer "B.Cu") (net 2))
 (segment (start 209 85.8) (end 208.948 85.852) (width 0.2) (layer "B.Cu") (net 2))
 (segment (start 217.678 85.852) (end 211.948 85.852) (width 0.2) (layer "B.Cu") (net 2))
 (segment (start 198.628 85.852) (end 198.628 91.428) (width 0.2) (layer "B.Cu") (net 2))
 (segment (start 229.388 68.326) (end 226.226 68.326) (width 0.2) (layer "B.Cu") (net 2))
 (segment (start 208.5 92.7) (end 211.8 92.7) (width 0.2) (layer "F.Cu") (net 8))
 (via (at 211.8 92.7) (size 0.6) (drill 0.3) (layers "F.Cu" "B.Cu") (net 8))
 (via (at 208.5 92.7) (size 0.6) (drill 0.3) (layers "F.Cu" "B.Cu") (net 8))
 (segment (start 205.1 92.7) (end 208.5 92.7) (width 0.2) (layer "B.Cu") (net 8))
 (segment (start 213.3 94.2) (end 218.9 94.2) (width 0.2) (layer "B.Cu") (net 8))
 (segment (start 211.8 92.7) (end 213.3 94.2) (width 0.2) (layer "B.Cu") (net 8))
 (segment (start 224.1 92.7) (end 224.9 92.7) (width 0.2) (layer "B.Cu") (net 7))
 (segment (start 226.4025 94.2025) (end 238.0125 94.2025) (width 0.2) (layer "B.Cu") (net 7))
 (segment (start 224.9 92.7) (end 226.4025 94.2025) (width 0.2) (layer "B.Cu") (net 7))
 (segment (start 244.0125 92.7025) (end 245.5125 94.2025) (width 0.2) (layer "B.Cu") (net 5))
 (segment (start 243.2125 92.7025) (end 244.0125 92.7025) (width 0.2) (layer "B.Cu") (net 5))
 (segment (start 245.5125 94.2025) (end 257.0125 94.2025) (width 0.2) (layer "B.Cu") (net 5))
 (segment (start 204.978 64.262) (end 204.978 83.312) (width 0.2) (layer "F.Cu") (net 11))
 (segment (start 198.12 57.404) (end 204.978 64.262) (width 0.2) (layer "F.Cu") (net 11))
 (segment (start 224.028 83.312) (end 222.212 83.312) (width 0.2) (layer "F.Cu") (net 1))
 (segment (start 204.378 65.5) (end 203.676 65.5) (width 0.2) (layer "F.Cu") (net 1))
 (segment (start 203.676 65.5) (end 198.12 59.944) (width 0.2) (layer "F.Cu") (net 1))
 (segment (start 222.212 83.312) (end 206.3 67.4) (width 0.2) (layer "F.Cu") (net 1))
 (via (at 206.3 67.4) (size 0.6) (drill 0.3) (layers "F.Cu" "B.Cu") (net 1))
 (via (at 204.378 65.5) (size 0.6) (drill 0.3) (layers "F.Cu" "B.Cu") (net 1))
 (segment (start 204.4 65.5) (end 204.378 65.5) (width 0.2) (layer "B.Cu") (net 1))
 (segment (start 206.3 67.4) (end 204.4 65.5) (width 0.2) (layer "B.Cu") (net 1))
 (segment (start 223.556 80.3) (end 213.36 70.104) (width 0.2) (layer "F.Cu") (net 9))
 (segment (start 240.066 80.3) (end 223.556 80.3) (width 0.2) (layer "F.Cu") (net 9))
 (segment (start 243.078 83.312) (end 240.066 80.3) (width 0.2) (layer "F.Cu") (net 9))
 (segment (start 257.316 78.5) (end 225.131 78.5) (width 0.2) (layer "F.Cu") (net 6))
 (segment (start 262.128 83.312) (end 257.316 78.5) (width 0.2) (layer "F.Cu") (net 6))
 (segment (start 225.131 78.5) (end 214.195 67.564) (width 0.2) (layer "F.Cu") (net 6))
 (segment (start 229.388 60.706) (end 226.133 63.961) (width 0.2) (layer "F.Cu") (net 14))
 (segment (start 201.4 64.6) (end 200.976 65.024) (width 0.2) (layer "F.Cu") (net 14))
 (segment (start 200.976 65.024) (end 197.285 65.024) (width 0.2) (layer "F.Cu") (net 14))
 (segment (start 206.839 63.961) (end 206.3 64.5) (width 0.2) (layer "F.Cu") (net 14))
 (segment (start 226.133 63.961) (end 206.839 63.961) (width 0.2) (layer "F.Cu") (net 14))
 (via (at 201.4 64.6) (size 0.6) (drill 0.3) (layers "F.Cu" "B.Cu") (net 14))
 (via (at 206.3 64.5) (size 0.6) (drill 0.3) (layers "F.Cu" "B.Cu") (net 14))
 (segment (start 206.3 64.5) (end 201.5 64.5) (width 0.2) (layer "B.Cu") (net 14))
 (segment (start 201.5 64.5) (end 201.4 64.6) (width 0.2) (layer "B.Cu") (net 14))
 (segment (start 209.999 66.501) (end 226.133 66.501) (width 0.2) (layer "F.Cu") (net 15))
 (segment (start 208.3 68.2) (end 209.999 66.501) (width 0.2) (layer "F.Cu") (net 15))
 (segment (start 203.064 67.564) (end 203.1 67.6) (width 0.2) (layer "F.Cu") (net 15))
 (segment (start 198.12 67.564) (end 203.064 67.564) (width 0.2) (layer "F.Cu") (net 15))
 (segment (start 226.133 66.501) (end 229.388 63.246) (width 0.2) (layer "F.Cu") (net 15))
 (via (at 208.3 68.2) (size 0.6) (drill 0.3) (layers "F.Cu" "B.Cu") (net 15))
 (via (at 203.1 67.6) (size 0.6) (drill 0.3) (layers "F.Cu" "B.Cu") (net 15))
 (segment (start 203.1 67.6) (end 203.7 68.2) (width 0.2) (layer "B.Cu") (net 15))
 (segment (start 203.7 68.2) (end 208.3 68.2) (width 0.2) (layer "B.Cu") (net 15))
 (segment (start 229.388 65.786) (end 223.546 59.944) (width 0.5) (layer "B.Cu") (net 22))
 (segment (start 223.546 59.944) (end 213.36 59.944) (width 0.5) (layer "B.Cu") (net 22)))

